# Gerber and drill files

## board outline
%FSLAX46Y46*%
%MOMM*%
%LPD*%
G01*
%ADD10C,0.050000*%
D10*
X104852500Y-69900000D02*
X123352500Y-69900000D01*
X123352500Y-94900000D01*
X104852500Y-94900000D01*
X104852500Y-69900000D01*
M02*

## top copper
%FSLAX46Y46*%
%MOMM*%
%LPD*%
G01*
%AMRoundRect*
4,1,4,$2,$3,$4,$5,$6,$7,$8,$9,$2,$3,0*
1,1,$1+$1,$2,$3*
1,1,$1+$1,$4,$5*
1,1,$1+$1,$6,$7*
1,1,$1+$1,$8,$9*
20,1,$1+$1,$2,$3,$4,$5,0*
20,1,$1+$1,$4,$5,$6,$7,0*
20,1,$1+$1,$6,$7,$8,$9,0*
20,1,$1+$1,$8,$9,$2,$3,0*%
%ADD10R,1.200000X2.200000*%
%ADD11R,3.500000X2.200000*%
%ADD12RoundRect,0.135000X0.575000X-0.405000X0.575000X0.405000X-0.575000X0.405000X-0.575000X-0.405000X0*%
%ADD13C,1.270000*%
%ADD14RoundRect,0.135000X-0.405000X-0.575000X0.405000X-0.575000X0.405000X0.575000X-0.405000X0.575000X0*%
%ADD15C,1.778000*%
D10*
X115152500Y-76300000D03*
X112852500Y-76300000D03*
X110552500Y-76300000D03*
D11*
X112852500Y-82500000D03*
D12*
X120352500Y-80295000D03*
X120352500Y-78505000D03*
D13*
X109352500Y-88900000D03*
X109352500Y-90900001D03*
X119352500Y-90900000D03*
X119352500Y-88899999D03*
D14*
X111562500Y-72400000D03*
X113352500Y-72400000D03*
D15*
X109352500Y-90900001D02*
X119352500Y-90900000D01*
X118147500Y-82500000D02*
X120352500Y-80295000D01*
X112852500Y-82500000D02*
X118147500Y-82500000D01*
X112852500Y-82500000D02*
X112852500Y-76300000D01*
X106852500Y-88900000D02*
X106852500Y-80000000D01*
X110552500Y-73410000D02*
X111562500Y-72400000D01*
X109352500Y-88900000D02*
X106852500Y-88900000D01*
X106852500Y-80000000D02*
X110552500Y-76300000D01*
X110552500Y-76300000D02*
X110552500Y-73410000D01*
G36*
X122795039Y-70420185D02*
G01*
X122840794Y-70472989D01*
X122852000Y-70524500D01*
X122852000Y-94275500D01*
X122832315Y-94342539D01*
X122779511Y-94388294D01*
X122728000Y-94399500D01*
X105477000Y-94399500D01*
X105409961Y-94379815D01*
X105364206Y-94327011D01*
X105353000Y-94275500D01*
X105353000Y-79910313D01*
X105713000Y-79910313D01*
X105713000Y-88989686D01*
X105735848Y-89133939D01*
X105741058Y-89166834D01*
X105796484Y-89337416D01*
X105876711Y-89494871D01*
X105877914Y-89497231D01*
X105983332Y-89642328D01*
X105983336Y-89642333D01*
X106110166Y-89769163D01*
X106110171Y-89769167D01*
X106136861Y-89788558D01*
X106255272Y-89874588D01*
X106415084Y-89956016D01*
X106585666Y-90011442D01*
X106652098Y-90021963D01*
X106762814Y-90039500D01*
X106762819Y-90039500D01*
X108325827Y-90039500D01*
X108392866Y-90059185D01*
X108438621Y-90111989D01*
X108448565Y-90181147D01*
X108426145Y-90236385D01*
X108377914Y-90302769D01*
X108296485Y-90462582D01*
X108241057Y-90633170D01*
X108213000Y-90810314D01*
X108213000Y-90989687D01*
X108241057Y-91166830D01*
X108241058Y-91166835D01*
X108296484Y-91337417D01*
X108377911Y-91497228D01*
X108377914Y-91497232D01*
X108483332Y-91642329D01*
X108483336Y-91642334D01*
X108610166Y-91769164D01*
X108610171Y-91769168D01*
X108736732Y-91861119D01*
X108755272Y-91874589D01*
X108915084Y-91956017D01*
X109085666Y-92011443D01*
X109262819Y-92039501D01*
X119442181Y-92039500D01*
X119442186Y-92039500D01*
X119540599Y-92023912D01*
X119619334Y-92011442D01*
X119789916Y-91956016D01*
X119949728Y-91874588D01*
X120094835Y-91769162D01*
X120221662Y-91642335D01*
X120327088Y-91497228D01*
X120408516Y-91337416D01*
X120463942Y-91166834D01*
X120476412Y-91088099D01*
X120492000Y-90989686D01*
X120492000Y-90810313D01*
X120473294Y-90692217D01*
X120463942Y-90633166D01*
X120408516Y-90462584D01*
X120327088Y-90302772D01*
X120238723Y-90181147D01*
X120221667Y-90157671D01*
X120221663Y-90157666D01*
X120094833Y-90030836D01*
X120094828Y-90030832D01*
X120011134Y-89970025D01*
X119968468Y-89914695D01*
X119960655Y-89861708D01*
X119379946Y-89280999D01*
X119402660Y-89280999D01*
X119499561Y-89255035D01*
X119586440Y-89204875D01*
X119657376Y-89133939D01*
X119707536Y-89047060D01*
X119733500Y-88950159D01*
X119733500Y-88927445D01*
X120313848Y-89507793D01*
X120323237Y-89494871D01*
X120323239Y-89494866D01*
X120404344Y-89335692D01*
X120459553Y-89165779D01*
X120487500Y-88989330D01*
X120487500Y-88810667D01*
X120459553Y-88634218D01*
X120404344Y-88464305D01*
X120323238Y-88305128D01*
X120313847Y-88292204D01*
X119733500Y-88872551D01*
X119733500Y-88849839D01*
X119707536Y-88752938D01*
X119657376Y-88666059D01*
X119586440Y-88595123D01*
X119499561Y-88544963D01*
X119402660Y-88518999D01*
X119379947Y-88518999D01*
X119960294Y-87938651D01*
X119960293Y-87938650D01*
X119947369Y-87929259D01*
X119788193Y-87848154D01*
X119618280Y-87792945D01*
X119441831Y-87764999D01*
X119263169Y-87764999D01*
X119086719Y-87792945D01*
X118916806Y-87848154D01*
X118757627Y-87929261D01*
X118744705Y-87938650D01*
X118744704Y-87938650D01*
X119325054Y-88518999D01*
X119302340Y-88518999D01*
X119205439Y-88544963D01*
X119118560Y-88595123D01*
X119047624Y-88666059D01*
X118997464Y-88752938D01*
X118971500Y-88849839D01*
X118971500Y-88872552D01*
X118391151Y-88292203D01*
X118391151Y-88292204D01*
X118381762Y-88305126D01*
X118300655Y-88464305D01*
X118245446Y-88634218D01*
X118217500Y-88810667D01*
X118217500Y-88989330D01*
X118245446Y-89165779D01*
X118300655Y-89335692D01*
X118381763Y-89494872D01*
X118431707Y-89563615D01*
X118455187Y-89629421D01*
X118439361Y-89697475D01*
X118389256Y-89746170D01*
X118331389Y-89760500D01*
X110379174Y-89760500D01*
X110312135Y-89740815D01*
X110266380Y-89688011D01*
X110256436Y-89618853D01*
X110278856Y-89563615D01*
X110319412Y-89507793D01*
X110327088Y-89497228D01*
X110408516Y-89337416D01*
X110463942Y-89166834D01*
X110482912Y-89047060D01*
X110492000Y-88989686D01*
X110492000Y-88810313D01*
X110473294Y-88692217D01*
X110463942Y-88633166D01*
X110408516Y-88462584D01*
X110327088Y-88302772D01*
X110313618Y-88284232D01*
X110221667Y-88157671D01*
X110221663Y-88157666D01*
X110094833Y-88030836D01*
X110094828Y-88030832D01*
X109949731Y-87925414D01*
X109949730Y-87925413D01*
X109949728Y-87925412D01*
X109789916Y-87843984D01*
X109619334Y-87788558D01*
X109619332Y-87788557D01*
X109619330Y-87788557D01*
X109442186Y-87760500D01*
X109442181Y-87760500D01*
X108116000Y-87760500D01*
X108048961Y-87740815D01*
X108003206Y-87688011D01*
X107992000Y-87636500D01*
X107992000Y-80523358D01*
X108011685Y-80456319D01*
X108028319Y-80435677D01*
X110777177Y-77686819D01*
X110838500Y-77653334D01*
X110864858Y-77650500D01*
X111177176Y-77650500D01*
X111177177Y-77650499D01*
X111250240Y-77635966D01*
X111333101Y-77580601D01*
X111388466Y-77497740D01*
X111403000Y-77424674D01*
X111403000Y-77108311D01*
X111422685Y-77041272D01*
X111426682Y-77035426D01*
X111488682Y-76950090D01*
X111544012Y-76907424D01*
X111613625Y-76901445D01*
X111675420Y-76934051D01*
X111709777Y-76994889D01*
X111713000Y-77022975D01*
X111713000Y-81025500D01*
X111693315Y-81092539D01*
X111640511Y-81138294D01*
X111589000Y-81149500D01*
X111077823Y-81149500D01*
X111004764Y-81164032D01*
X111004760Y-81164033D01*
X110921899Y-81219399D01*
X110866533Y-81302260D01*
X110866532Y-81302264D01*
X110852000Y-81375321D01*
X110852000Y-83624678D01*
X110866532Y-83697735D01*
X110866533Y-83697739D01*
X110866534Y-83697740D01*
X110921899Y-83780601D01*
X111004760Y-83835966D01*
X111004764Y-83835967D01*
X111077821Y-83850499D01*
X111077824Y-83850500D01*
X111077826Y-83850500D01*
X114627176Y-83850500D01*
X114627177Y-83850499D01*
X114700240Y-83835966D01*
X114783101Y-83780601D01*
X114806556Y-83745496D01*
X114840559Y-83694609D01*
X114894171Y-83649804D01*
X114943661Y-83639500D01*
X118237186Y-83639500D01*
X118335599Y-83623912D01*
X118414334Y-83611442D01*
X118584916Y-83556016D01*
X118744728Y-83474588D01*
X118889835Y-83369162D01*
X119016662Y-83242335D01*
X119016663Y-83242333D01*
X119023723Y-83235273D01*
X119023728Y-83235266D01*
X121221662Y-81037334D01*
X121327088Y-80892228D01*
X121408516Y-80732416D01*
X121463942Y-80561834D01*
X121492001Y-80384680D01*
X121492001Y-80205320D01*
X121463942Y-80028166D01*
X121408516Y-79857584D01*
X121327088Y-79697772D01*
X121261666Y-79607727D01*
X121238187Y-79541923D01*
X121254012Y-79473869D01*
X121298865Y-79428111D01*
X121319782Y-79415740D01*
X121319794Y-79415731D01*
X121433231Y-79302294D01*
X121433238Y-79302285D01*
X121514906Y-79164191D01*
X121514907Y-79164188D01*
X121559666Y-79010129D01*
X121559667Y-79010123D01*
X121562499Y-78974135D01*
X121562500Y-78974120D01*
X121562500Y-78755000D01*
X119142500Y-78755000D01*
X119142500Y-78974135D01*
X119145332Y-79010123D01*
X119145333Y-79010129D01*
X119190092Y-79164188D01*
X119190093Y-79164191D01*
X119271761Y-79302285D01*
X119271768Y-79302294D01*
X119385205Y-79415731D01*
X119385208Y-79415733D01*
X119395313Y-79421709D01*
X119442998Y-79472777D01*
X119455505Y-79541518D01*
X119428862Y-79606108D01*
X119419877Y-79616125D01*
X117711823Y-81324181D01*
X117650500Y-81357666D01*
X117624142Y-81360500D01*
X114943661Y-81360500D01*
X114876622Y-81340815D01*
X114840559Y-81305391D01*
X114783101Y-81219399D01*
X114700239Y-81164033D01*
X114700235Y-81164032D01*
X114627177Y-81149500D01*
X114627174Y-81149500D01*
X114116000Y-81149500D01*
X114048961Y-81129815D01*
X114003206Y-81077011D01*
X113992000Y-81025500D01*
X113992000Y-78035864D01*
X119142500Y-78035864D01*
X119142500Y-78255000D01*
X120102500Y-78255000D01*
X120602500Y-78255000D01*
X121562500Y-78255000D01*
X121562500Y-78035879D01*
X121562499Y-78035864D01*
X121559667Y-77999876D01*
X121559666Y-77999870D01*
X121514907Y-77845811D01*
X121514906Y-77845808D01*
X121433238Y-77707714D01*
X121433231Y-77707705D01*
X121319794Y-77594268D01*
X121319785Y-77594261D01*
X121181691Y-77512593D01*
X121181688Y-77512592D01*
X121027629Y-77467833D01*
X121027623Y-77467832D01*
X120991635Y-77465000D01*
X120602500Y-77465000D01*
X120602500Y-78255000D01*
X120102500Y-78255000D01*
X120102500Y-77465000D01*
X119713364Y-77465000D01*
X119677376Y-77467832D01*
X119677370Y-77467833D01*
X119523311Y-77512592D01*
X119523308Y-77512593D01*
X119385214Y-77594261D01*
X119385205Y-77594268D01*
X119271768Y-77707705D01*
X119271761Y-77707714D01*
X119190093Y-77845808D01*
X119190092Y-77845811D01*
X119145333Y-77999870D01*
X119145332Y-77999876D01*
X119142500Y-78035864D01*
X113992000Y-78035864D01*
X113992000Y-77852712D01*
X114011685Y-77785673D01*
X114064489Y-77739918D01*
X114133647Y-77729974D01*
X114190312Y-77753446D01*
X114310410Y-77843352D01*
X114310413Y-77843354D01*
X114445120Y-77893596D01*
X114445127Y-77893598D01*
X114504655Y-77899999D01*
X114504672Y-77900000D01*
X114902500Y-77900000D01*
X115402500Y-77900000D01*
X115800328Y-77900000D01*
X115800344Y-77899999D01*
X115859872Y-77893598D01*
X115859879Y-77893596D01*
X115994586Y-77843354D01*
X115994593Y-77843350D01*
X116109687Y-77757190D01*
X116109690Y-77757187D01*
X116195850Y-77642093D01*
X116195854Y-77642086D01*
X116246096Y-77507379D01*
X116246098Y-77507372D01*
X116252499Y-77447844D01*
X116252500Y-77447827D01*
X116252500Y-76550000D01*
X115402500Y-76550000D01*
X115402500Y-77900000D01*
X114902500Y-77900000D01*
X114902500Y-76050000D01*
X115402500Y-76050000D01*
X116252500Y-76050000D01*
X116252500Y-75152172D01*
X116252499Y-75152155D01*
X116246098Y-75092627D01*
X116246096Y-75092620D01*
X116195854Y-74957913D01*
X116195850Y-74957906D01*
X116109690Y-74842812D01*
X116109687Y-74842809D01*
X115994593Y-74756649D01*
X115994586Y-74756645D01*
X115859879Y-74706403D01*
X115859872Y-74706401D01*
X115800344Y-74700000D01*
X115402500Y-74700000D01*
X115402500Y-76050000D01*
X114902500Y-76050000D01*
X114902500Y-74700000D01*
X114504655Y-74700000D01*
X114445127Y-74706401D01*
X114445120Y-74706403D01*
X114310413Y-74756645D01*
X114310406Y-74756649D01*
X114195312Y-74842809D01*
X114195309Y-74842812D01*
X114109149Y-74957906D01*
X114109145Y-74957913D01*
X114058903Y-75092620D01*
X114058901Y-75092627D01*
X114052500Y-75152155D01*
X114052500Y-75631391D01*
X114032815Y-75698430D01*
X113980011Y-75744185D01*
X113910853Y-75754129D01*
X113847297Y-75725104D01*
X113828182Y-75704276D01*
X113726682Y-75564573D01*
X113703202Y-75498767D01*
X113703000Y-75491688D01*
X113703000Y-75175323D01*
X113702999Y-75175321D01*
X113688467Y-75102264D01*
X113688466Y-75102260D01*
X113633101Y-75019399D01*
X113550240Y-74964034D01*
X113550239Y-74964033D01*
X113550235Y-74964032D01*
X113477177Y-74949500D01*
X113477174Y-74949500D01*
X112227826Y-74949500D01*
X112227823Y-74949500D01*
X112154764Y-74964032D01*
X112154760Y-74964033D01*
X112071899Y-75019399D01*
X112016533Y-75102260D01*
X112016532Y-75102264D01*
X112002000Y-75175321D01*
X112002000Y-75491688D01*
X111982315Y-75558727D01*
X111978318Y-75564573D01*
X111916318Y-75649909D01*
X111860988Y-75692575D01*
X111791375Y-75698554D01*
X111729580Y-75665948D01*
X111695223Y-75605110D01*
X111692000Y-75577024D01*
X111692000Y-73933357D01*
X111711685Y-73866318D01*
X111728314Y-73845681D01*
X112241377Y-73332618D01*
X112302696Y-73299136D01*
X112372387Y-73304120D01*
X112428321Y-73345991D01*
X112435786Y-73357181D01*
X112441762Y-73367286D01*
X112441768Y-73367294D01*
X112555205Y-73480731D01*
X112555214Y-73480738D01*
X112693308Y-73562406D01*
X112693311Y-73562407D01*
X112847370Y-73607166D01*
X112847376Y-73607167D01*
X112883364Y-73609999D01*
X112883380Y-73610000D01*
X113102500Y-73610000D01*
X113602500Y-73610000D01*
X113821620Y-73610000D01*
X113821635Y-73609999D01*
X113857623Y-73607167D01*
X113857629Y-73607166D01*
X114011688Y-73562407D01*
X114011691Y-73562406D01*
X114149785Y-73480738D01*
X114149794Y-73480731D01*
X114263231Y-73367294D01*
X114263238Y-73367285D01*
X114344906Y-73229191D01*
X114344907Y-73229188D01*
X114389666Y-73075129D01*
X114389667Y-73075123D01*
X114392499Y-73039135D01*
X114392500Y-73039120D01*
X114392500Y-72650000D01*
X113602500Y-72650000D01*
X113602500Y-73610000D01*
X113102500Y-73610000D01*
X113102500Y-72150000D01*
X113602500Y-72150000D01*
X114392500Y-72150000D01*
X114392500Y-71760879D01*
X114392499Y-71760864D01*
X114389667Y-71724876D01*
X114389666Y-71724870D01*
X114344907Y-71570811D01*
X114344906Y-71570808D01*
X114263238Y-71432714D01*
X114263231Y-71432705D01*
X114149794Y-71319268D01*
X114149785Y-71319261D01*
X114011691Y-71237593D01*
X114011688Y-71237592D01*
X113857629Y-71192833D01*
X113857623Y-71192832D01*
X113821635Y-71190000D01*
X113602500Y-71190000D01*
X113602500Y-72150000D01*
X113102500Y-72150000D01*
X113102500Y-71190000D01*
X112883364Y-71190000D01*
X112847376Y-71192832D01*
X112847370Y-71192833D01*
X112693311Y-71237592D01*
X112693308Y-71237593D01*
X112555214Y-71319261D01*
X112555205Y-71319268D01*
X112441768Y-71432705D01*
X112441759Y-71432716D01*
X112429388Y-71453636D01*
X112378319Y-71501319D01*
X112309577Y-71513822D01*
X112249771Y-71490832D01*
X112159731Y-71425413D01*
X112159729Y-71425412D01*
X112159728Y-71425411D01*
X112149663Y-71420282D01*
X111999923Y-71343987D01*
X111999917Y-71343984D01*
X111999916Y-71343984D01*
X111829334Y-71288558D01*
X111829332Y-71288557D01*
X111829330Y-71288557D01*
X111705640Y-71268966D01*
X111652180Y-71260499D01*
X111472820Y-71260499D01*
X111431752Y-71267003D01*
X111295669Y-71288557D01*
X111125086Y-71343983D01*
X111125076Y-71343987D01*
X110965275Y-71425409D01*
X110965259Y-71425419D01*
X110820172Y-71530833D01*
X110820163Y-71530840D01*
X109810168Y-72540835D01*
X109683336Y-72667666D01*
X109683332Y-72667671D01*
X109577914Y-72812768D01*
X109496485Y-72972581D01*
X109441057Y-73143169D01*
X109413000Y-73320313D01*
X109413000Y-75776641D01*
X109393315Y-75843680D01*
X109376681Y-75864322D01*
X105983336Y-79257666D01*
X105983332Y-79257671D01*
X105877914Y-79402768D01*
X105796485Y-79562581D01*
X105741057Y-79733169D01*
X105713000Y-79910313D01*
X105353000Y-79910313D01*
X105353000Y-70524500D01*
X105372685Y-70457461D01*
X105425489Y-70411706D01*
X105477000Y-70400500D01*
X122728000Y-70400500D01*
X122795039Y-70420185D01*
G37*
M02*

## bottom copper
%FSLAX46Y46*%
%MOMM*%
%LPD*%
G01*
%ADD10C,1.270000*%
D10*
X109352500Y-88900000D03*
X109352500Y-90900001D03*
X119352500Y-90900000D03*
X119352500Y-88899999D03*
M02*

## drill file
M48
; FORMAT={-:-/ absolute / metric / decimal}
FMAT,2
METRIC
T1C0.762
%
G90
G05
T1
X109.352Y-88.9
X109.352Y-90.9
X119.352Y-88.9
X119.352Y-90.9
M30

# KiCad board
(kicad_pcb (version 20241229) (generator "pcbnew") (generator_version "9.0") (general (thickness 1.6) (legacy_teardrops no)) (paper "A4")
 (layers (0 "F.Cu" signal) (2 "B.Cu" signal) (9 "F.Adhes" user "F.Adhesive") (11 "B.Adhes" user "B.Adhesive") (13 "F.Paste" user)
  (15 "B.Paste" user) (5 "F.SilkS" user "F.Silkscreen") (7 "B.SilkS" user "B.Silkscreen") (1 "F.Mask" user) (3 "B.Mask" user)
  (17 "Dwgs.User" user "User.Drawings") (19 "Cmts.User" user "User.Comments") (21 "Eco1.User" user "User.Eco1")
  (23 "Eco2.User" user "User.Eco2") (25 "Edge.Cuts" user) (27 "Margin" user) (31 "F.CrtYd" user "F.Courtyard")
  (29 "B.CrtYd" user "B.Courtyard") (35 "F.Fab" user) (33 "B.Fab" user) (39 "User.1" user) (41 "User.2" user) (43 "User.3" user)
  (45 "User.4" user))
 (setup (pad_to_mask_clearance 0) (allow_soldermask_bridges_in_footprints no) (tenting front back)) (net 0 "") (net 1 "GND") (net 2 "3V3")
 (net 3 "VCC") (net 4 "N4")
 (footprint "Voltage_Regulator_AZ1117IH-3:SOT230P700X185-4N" (layer "F.Cu") (at 112.8525 79.4 -90)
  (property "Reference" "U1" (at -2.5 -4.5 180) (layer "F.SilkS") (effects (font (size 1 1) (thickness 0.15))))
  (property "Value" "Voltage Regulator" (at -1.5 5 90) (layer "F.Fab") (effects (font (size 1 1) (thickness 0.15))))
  (pad "1" smd rect (at -3.1 -2.3 270) (size 2.2 1.2) (layers "F.Cu" "F.Mask" "F.Paste") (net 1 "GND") (solder_mask_margin 0.102))
  (pad "2" smd rect (at -3.1 0 270) (size 2.2 1.2) (layers "F.Cu" "F.Mask" "F.Paste") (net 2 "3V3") (solder_mask_margin 0.102))
  (pad "3" smd rect (at -3.1 2.3 270) (size 2.2 1.2) (layers "F.Cu" "F.Mask" "F.Paste") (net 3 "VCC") (solder_mask_margin 0.102))
  (pad "4" smd rect (at 3.1 0 270) (size 2.2 3.5) (layers "F.Cu" "F.Mask" "F.Paste") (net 2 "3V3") (solder_mask_margin 0.102)))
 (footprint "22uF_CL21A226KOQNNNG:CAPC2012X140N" (layer "F.Cu") (at 120.3525 79.4 90)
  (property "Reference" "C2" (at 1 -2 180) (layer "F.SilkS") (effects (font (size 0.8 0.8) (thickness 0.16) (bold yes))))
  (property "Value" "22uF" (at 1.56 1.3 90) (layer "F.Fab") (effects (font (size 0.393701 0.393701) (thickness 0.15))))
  (pad "1" smd roundrect (at -0.895 0 90) (size 1.08 1.42) (layers "F.Cu" "F.Mask" "F.Paste") (roundrect_rratio 0.125) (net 2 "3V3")
   (solder_mask_margin 0.102))
  (pad "2" smd roundrect (at 0.895 0 90) (size 1.08 1.42) (layers "F.Cu" "F.Mask" "F.Paste") (roundrect_rratio 0.125) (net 1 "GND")
   (solder_mask_margin 0.102)))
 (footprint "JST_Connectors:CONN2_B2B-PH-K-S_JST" (layer "F.Cu") (at 109.3525 88.9 90)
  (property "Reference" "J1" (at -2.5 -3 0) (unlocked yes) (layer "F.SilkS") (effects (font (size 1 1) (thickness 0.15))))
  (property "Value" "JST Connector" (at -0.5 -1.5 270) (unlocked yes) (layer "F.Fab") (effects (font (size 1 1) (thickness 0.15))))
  (pad "1" thru_hole circle (at 0 0 90) (size 1.27 1.27) (drill 0.762) (layers "*.Cu" "*.Mask") (remove_unused_layers no) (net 3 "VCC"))
  (pad "2" thru_hole circle (at -2.000001 0 90) (size 1.27 1.27) (drill 0.762) (layers "*.Cu" "*.Mask") (remove_unused_layers no)
   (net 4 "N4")))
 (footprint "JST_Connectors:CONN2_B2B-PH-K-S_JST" (layer "F.Cu") (at 119.3525 90.9 -90)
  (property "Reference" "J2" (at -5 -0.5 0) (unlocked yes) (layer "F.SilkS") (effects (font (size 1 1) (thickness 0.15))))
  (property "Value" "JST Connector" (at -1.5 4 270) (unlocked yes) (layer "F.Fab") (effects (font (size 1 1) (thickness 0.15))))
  (pad "1" thru_hole circle (at 0 0 270) (size 1.27 1.27) (drill 0.762) (layers "*.Cu" "*.Mask") (remove_unused_layers no) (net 4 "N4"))
  (pad "2" thru_hole circle (at -2.000001 0 270) (size 1.27 1.27) (drill 0.762) (layers "*.Cu" "*.Mask") (remove_unused_layers no)
   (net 1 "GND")))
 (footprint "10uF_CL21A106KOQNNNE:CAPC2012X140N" (layer "F.Cu") (at 112.4575 72.4)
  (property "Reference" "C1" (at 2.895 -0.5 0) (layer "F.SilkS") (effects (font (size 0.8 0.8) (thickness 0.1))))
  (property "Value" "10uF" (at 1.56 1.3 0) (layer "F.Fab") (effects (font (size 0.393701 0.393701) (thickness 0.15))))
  (pad "1" smd roundrect (at -0.895 0) (size 1.08 1.42) (layers "F.Cu" "F.Mask" "F.Paste") (roundrect_rratio 0.125) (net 3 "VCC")
   (solder_mask_margin 0.102))
  (pad "2" smd roundrect (at 0.895 0) (size 1.08 1.42) (layers "F.Cu" "F.Mask" "F.Paste") (roundrect_rratio 0.125) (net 1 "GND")
   (solder_mask_margin 0.102)))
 (gr_rect (start 104.8525 69.9) (end 123.3525 94.9) (stroke (width 0.05) (type default)) (fill no) (layer "Edge.Cuts"))
 (segment (start 109.3525 90.900001) (end 119.3525 90.9) (width 1.778) (layer "F.Cu") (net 4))
 (segment (start 118.1475 82.5) (end 120.3525 80.295) (width 1.778) (layer "F.Cu") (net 2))
 (segment (start 112.8525 82.5) (end 118.1475 82.5) (width 1.778) (layer "F.Cu") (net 2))
 (segment (start 112.8525 82.5) (end 112.8525 76.3) (width 1.778) (layer "F.Cu") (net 2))
 (segment (start 106.8525 88.9) (end 106.8525 80) (width 1.778) (layer "F.Cu") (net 3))
 (segment (start 110.5525 73.41) (end 111.5625 72.4) (width 1.778) (layer "F.Cu") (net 3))
 (segment (start 109.3525 88.9) (end 106.8525 88.9) (width 1.778) (layer "F.Cu") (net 3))
 (segment (start 106.8525 80) (end 110.5525 76.3) (width 1.778) (layer "F.Cu") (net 3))
 (segment (start 110.5525 76.3) (end 110.5525 73.41) (width 1.778) (layer "F.Cu") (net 3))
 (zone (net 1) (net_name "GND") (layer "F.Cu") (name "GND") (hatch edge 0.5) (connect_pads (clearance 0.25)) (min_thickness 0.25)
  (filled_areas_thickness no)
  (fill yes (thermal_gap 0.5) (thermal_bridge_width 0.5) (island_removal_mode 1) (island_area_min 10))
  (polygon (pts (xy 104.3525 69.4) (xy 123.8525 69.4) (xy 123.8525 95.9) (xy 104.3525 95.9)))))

